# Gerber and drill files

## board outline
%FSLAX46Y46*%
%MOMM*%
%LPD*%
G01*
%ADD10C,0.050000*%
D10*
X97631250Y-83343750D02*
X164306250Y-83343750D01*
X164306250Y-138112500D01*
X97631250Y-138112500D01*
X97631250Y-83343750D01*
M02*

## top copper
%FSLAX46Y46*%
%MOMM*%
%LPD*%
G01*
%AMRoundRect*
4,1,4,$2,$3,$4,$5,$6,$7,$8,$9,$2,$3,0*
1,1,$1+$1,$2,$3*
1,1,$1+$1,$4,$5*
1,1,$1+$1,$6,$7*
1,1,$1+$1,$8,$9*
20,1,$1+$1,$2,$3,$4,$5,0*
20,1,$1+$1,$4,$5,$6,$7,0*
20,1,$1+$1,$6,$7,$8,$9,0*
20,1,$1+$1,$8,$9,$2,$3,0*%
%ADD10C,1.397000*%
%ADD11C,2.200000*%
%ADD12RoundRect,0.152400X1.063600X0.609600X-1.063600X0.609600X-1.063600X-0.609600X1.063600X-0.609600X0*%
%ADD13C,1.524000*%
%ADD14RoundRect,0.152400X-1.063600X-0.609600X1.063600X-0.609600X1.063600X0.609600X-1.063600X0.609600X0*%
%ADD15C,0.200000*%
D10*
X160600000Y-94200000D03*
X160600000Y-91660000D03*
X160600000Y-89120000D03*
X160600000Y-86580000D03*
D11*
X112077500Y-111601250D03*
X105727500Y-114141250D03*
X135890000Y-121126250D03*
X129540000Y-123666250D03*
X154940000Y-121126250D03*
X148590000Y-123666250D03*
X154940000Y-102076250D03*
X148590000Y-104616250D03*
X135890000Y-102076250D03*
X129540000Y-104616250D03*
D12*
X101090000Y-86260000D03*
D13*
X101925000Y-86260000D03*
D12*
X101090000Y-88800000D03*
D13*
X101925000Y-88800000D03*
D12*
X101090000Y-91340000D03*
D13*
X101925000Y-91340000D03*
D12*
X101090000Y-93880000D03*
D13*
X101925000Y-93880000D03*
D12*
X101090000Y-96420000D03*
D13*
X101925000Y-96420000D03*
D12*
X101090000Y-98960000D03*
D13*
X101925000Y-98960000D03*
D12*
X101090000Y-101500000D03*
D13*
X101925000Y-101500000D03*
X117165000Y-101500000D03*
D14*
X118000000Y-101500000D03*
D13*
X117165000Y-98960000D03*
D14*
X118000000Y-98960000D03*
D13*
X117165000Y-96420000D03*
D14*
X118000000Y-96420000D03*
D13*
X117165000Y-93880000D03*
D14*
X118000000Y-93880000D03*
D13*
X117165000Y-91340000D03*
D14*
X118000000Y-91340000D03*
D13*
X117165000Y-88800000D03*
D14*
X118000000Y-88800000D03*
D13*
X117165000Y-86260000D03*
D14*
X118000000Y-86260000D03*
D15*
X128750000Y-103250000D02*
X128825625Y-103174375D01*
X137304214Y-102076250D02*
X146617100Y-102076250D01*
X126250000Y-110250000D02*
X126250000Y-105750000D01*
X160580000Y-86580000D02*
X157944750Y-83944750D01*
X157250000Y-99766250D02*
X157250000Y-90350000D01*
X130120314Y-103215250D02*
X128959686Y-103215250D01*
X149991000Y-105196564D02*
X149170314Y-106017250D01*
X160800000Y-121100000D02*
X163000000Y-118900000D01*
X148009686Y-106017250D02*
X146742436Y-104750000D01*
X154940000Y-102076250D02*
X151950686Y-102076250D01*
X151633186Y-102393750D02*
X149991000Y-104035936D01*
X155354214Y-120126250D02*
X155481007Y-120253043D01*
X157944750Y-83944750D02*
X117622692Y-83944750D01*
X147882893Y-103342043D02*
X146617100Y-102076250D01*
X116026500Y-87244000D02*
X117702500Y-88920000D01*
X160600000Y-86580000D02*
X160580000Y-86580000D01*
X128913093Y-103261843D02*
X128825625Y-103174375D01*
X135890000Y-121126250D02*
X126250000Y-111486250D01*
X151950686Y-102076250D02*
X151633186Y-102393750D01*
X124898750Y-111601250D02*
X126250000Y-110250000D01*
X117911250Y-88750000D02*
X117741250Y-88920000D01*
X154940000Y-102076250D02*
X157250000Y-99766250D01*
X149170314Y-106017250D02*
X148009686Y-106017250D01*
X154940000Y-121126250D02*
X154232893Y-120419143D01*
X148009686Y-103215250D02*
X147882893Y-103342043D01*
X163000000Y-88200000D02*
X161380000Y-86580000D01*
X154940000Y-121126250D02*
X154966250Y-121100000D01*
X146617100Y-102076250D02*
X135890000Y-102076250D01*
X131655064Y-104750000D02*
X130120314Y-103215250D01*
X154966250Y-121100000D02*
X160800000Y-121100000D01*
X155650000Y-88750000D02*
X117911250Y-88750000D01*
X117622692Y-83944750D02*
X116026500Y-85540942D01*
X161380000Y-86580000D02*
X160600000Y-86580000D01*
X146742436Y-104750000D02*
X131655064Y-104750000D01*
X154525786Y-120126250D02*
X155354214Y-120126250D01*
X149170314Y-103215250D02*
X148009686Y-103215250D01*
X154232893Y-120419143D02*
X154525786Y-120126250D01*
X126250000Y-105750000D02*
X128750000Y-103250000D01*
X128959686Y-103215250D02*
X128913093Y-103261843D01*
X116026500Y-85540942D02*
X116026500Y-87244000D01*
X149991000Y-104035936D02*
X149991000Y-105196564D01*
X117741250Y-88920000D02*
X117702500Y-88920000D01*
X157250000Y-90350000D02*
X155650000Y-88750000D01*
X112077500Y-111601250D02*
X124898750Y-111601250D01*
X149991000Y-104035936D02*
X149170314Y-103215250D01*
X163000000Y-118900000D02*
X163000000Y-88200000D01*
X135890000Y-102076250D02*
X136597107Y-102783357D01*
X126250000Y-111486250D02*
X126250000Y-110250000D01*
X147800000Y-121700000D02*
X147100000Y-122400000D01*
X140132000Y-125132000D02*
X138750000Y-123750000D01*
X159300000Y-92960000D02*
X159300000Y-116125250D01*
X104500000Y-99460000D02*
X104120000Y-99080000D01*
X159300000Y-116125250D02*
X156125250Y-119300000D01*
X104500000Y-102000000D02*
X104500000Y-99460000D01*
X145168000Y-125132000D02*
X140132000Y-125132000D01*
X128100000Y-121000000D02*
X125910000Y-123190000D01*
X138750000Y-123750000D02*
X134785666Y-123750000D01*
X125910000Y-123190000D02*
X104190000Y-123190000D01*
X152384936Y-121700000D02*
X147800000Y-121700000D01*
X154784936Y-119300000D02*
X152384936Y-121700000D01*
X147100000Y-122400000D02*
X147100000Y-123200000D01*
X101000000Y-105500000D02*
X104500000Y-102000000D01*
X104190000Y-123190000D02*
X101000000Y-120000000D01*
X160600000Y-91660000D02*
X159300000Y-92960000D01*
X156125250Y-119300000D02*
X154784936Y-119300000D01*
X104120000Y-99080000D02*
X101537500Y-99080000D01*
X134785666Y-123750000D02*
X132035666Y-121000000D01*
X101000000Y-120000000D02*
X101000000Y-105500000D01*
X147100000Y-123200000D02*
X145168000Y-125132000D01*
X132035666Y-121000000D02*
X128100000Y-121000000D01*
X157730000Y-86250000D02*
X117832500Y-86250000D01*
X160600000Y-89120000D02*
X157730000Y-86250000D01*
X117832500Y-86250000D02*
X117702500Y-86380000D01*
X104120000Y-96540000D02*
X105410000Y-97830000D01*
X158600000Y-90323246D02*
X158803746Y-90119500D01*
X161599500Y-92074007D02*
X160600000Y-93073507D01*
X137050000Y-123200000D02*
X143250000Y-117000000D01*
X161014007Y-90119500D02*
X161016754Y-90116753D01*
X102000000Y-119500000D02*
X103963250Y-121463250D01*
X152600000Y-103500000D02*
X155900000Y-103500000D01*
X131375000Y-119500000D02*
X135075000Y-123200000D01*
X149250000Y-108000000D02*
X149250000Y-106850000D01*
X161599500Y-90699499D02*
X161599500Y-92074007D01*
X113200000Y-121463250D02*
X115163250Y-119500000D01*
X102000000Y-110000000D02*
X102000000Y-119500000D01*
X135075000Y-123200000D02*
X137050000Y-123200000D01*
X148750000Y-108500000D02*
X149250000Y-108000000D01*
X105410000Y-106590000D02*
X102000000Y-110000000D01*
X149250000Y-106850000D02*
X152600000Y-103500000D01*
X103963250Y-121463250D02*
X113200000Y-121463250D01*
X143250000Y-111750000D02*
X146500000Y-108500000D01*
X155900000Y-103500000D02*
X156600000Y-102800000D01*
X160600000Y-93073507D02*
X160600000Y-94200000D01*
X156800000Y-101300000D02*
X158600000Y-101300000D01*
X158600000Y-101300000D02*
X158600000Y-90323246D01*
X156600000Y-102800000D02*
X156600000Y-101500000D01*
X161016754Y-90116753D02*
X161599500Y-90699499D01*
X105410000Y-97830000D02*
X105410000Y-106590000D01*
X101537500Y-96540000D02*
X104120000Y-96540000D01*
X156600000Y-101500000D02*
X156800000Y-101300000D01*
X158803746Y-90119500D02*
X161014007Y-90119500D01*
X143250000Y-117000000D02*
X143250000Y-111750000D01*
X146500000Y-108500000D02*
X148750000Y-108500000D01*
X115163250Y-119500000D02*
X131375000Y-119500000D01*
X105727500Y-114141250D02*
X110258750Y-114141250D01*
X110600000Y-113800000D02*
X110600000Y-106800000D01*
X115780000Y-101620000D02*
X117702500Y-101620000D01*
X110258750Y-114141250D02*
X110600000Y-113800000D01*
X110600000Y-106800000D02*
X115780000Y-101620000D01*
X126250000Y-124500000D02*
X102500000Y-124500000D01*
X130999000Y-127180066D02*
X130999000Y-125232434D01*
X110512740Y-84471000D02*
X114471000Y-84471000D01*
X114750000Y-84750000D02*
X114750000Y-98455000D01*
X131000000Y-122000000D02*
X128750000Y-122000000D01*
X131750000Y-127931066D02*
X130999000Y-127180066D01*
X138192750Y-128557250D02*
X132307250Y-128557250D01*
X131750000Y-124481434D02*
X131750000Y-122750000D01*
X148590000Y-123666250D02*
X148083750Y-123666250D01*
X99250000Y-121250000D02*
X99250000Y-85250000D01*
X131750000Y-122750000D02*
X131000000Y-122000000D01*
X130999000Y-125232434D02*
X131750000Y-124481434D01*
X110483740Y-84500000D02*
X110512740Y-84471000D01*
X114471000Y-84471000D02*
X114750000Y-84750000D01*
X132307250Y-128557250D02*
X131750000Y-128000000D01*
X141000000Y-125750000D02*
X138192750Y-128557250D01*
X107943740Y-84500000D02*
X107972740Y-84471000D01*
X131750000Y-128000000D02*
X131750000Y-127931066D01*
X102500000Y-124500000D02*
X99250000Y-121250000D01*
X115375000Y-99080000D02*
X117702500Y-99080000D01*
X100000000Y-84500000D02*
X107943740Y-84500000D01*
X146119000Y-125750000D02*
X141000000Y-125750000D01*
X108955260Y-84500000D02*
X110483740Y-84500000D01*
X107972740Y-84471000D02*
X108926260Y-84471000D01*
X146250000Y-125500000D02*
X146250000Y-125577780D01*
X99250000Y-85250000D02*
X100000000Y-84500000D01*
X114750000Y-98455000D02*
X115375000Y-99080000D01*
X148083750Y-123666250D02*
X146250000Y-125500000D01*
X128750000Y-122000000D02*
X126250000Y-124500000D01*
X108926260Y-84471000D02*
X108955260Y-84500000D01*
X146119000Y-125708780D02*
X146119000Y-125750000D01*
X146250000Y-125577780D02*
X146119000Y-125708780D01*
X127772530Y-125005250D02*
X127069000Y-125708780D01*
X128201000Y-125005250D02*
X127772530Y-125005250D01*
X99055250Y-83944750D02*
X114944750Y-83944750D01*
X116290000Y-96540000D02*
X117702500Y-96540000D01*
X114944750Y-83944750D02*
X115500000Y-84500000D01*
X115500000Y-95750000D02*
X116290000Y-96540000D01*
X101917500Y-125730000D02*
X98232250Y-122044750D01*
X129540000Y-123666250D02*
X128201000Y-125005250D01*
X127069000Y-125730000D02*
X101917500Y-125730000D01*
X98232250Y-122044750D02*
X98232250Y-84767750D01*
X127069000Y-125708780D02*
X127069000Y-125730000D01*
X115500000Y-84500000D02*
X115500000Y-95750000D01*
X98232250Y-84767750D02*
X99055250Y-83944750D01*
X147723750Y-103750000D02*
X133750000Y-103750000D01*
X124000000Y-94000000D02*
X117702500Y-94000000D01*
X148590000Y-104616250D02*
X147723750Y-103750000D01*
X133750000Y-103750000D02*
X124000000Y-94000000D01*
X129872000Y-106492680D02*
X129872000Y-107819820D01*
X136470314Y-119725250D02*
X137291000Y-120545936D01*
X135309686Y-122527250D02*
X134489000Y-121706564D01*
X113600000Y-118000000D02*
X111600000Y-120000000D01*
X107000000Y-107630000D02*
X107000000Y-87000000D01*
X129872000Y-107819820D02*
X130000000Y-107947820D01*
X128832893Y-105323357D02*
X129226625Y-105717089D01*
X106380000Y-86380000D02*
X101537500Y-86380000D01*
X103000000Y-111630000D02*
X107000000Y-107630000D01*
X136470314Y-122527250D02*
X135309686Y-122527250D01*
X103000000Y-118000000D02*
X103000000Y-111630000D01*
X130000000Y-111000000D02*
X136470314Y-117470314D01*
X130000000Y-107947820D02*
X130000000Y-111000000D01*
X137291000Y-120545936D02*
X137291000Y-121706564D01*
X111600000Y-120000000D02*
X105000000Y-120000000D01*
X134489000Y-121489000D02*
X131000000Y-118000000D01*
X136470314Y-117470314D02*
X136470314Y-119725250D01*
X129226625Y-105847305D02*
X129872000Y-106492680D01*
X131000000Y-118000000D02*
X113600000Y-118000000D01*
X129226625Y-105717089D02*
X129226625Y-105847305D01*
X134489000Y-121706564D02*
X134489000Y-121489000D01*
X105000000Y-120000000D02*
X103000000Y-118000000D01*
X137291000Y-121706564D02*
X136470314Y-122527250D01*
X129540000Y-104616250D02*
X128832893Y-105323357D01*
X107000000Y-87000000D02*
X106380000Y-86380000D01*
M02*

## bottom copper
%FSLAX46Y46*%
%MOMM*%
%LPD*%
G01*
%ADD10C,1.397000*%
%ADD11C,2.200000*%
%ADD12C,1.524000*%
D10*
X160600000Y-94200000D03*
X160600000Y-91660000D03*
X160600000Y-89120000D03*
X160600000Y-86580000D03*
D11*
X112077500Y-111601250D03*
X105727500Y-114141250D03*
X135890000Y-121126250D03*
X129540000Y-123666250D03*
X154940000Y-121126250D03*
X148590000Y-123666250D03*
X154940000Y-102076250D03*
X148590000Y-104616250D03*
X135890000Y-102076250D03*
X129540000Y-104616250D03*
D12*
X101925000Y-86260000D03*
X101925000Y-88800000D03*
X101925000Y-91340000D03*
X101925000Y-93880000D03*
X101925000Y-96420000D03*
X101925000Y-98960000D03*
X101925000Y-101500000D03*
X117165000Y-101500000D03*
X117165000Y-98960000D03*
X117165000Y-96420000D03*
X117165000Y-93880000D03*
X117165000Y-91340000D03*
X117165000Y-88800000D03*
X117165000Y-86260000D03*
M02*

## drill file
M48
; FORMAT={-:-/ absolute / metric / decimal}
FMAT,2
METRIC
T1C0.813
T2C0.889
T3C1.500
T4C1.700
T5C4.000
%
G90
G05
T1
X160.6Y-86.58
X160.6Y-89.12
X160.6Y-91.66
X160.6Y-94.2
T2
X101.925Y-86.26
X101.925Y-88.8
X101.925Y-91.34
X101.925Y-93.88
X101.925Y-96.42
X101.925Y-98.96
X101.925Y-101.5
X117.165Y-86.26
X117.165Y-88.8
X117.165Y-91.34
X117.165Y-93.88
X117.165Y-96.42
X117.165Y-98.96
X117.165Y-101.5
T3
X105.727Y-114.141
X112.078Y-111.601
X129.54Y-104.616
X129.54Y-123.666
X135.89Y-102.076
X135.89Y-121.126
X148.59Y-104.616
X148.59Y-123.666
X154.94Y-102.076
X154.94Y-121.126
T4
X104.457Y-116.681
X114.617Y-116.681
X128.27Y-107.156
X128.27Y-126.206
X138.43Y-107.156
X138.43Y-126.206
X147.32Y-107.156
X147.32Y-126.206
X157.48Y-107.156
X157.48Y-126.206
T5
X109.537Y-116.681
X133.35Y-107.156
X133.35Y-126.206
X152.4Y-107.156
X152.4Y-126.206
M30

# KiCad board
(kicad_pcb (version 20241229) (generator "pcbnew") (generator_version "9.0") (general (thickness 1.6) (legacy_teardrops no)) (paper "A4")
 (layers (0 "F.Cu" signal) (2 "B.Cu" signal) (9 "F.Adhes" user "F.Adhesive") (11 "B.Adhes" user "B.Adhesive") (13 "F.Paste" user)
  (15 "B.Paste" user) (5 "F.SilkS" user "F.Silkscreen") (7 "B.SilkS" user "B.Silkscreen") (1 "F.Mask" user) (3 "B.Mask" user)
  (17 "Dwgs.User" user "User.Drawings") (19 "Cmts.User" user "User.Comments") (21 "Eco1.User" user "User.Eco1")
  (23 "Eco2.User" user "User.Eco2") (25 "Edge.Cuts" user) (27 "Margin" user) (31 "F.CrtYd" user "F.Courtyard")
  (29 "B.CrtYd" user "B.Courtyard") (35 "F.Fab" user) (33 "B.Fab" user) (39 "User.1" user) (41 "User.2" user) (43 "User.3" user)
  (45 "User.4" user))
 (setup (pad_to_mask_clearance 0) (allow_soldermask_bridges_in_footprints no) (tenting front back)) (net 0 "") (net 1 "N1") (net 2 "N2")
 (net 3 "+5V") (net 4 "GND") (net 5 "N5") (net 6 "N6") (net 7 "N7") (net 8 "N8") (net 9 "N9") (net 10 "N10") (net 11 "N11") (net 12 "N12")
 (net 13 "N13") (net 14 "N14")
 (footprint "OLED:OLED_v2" (layer "F.Cu") (at 160.6 90.39 90)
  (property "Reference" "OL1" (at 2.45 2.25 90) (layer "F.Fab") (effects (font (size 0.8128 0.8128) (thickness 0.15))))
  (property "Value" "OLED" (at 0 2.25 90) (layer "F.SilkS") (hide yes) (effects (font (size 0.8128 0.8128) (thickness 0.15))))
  (pad "1" thru_hole circle (at -3.81 0 90) (size 1.397 1.397) (drill 0.8128) (layers "*.Cu" "B.Mask" "F.SilkS") (remove_unused_layers no)
   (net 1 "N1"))
  (pad "2" thru_hole circle (at -1.27 0 90) (size 1.397 1.397) (drill 0.8128) (layers "*.Cu" "B.Mask" "F.SilkS") (remove_unused_layers no)
   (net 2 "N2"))
  (pad "3" thru_hole circle (at 1.27 0 90) (size 1.397 1.397) (drill 0.8128) (layers "*.Cu" "B.Mask" "F.SilkS") (remove_unused_layers no)
   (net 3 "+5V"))
  (pad "4" thru_hole circle (at 3.81 0 90) (size 1.397 1.397) (drill 0.8128) (layers "*.Cu" "B.Mask" "F.SilkS") (remove_unused_layers no)
   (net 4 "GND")))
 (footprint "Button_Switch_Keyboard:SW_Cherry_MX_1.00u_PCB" (layer "F.Cu") (at 112.0775 111.60125)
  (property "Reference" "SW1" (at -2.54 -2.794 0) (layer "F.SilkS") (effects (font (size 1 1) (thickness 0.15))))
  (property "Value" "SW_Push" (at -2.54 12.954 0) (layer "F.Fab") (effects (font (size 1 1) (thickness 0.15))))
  (pad "" np_thru_hole circle (at -7.62 5.08) (size 1.7 1.7) (drill 1.7) (layers "*.Cu" "*.Mask"))
  (pad "" np_thru_hole circle (at -2.54 5.08) (size 4 4) (drill 4) (layers "*.Cu" "*.Mask"))
  (pad "" np_thru_hole circle (at 2.54 5.08) (size 1.7 1.7) (drill 1.7) (layers "*.Cu" "*.Mask"))
  (pad "1" thru_hole circle (at 0 0) (size 2.2 2.2) (drill 1.5) (layers "*.Cu" "*.Mask") (remove_unused_layers no) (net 4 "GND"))
  (pad "2" thru_hole circle (at -6.35 2.54) (size 2.2 2.2) (drill 1.5) (layers "*.Cu" "*.Mask") (remove_unused_layers no) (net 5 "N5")))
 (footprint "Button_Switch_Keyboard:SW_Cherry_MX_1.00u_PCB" (layer "F.Cu") (at 135.89 121.12625)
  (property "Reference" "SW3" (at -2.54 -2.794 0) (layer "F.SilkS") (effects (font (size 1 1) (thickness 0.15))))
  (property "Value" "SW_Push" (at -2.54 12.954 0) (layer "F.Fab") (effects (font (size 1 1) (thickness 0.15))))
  (pad "" np_thru_hole circle (at -7.62 5.08) (size 1.7 1.7) (drill 1.7) (layers "*.Cu" "*.Mask"))
  (pad "" np_thru_hole circle (at -2.54 5.08) (size 4 4) (drill 4) (layers "*.Cu" "*.Mask"))
  (pad "" np_thru_hole circle (at 2.54 5.08) (size 1.7 1.7) (drill 1.7) (layers "*.Cu" "*.Mask"))
  (pad "1" thru_hole circle (at 0 0) (size 2.2 2.2) (drill 1.5) (layers "*.Cu" "*.Mask") (remove_unused_layers no) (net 4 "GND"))
  (pad "2" thru_hole circle (at -6.35 2.54) (size 2.2 2.2) (drill 1.5) (layers "*.Cu" "*.Mask") (remove_unused_layers no) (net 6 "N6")))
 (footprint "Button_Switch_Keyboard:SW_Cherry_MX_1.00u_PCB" (layer "F.Cu") (at 154.94 121.12625)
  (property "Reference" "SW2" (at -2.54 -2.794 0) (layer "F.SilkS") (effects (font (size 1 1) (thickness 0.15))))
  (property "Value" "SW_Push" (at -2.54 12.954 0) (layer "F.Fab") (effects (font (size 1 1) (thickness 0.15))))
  (pad "" np_thru_hole circle (at -7.62 5.08) (size 1.7 1.7) (drill 1.7) (layers "*.Cu" "*.Mask"))
  (pad "" np_thru_hole circle (at -2.54 5.08) (size 4 4) (drill 4) (layers "*.Cu" "*.Mask"))
  (pad "" np_thru_hole circle (at 2.54 5.08) (size 1.7 1.7) (drill 1.7) (layers "*.Cu" "*.Mask"))
  (pad "1" thru_hole circle (at 0 0) (size 2.2 2.2) (drill 1.5) (layers "*.Cu" "*.Mask") (remove_unused_layers no) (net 4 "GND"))
  (pad "2" thru_hole circle (at -6.35 2.54) (size 2.2 2.2) (drill 1.5) (layers "*.Cu" "*.Mask") (remove_unused_layers no) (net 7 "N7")))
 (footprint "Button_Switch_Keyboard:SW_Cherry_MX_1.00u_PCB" (layer "F.Cu") (at 154.94 102.07625)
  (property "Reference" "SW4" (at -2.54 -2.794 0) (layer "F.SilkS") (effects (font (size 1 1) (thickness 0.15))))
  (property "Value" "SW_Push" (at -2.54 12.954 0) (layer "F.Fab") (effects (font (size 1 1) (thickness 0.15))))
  (pad "" np_thru_hole circle (at -7.62 5.08) (size 1.7 1.7) (drill 1.7) (layers "*.Cu" "*.Mask"))
  (pad "" np_thru_hole circle (at -2.54 5.08) (size 4 4) (drill 4) (layers "*.Cu" "*.Mask"))
  (pad "" np_thru_hole circle (at 2.54 5.08) (size 1.7 1.7) (drill 1.7) (layers "*.Cu" "*.Mask"))
  (pad "1" thru_hole circle (at 0 0) (size 2.2 2.2) (drill 1.5) (layers "*.Cu" "*.Mask") (remove_unused_layers no) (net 4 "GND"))
  (pad "2" thru_hole circle (at -6.35 2.54) (size 2.2 2.2) (drill 1.5) (layers "*.Cu" "*.Mask") (remove_unused_layers no) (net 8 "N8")))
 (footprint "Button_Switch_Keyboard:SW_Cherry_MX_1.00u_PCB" (layer "F.Cu") (at 135.89 102.07625)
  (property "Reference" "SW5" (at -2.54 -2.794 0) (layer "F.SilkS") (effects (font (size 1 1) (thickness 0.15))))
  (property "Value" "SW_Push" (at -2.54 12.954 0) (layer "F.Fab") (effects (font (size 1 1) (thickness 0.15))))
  (pad "" np_thru_hole circle (at -7.62 5.08) (size 1.7 1.7) (drill 1.7) (layers "*.Cu" "*.Mask"))
  (pad "" np_thru_hole circle (at -2.54 5.08) (size 4 4) (drill 4) (layers "*.Cu" "*.Mask"))
  (pad "" np_thru_hole circle (at 2.54 5.08) (size 1.7 1.7) (drill 1.7) (layers "*.Cu" "*.Mask"))
  (pad "1" thru_hole circle (at 0 0) (size 2.2 2.2) (drill 1.5) (layers "*.Cu" "*.Mask") (remove_unused_layers no) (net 4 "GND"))
  (pad "2" thru_hole circle (at -6.35 2.54) (size 2.2 2.2) (drill 1.5) (layers "*.Cu" "*.Mask") (remove_unused_layers no) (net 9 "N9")))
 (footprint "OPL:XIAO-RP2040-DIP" (layer "F.Cu") (at 109.545 93.88)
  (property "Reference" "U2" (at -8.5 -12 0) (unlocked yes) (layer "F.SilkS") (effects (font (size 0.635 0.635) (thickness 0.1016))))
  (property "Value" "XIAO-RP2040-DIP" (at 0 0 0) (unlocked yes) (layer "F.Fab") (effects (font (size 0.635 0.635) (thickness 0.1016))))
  (pad "1" smd roundrect (at -8.455 -7.62 180) (size 2.432 1.524) (layers "F.Cu" "F.Mask") (roundrect_rratio 0.1) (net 9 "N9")
   (thermal_bridge_angle 45))
  (pad "1" thru_hole circle (at -7.62 -7.62 180) (size 1.524 1.524) (drill 0.889) (layers "*.Cu" "*.Mask") (remove_unused_layers no)
   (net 9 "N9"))
  (pad "2" smd roundrect (at -8.455 -5.08 180) (size 2.432 1.524) (layers "F.Cu" "F.Mask") (roundrect_rratio 0.1) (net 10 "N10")
   (thermal_bridge_angle 45))
  (pad "2" thru_hole circle (at -7.62 -5.08 180) (size 1.524 1.524) (drill 0.889) (layers "*.Cu" "*.Mask") (remove_unused_layers no)
   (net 10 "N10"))
  (pad "3" smd roundrect (at -8.455 -2.54 180) (size 2.432 1.524) (layers "F.Cu" "F.Mask") (roundrect_rratio 0.1) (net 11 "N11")
   (thermal_bridge_angle 45))
  (pad "3" thru_hole circle (at -7.62 -2.54 180) (size 1.524 1.524) (drill 0.889) (layers "*.Cu" "*.Mask") (remove_unused_layers no)
   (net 11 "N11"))
  (pad "4" smd roundrect (at -8.455 0 180) (size 2.432 1.524) (layers "F.Cu" "F.Mask") (roundrect_rratio 0.1) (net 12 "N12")
   (thermal_bridge_angle 45))
  (pad "4" thru_hole circle (at -7.62 0 180) (size 1.524 1.524) (drill 0.889) (layers "*.Cu" "*.Mask") (remove_unused_layers no)
   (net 12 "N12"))
  (pad "5" smd roundrect (at -8.455 2.54 180) (size 2.432 1.524) (layers "F.Cu" "F.Mask") (roundrect_rratio 0.1) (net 1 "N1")
   (thermal_bridge_angle 45))
  (pad "5" thru_hole circle (at -7.62 2.54 180) (size 1.524 1.524) (drill 0.889) (layers "*.Cu" "*.Mask") (remove_unused_layers no)
   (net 1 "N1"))
  (pad "6" smd roundrect (at -8.455 5.08 180) (size 2.432 1.524) (layers "F.Cu" "F.Mask") (roundrect_rratio 0.1) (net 2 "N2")
   (thermal_bridge_angle 45))
  (pad "6" thru_hole circle (at -7.62 5.08 180) (size 1.524 1.524) (drill 0.889) (layers "*.Cu" "*.Mask") (remove_unused_layers no)
   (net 2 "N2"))
  (pad "7" smd roundrect (at -8.455 7.62 180) (size 2.432 1.524) (layers "F.Cu" "F.Mask") (roundrect_rratio 0.1) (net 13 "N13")
   (thermal_bridge_angle 45))
  (pad "7" thru_hole circle (at -7.62 7.62 180) (size 1.524 1.524) (drill 0.889) (layers "*.Cu" "*.Mask") (remove_unused_layers no)
   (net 13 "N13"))
  (pad "8" thru_hole circle (at 7.62 7.62) (size 1.524 1.524) (drill 0.889) (layers "*.Cu" "*.Mask") (remove_unused_layers no) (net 5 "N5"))
  (pad "8" smd roundrect (at 8.455 7.62) (size 2.432 1.524) (layers "F.Cu" "F.Mask") (roundrect_rratio 0.1) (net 5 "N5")
   (thermal_bridge_angle 45))
  (pad "9" thru_hole circle (at 7.62 5.08) (size 1.524 1.524) (drill 0.889) (layers "*.Cu" "*.Mask") (remove_unused_layers no) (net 7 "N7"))
  (pad "9" smd roundrect (at 8.455 5.08) (size 2.432 1.524) (layers "F.Cu" "F.Mask") (roundrect_rratio 0.1) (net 7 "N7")
   (thermal_bridge_angle 45))
  (pad "10" thru_hole circle (at 7.62 2.54) (size 1.524 1.524) (drill 0.889) (layers "*.Cu" "*.Mask") (remove_unused_layers no) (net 6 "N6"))
  (pad "10" smd roundrect (at 8.455 2.54) (size 2.432 1.524) (layers "F.Cu" "F.Mask") (roundrect_rratio 0.1) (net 6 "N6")
   (thermal_bridge_angle 45))
  (pad "11" thru_hole circle (at 7.62 0) (size 1.524 1.524) (drill 0.889) (layers "*.Cu" "*.Mask") (remove_unused_layers no) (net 8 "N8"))
  (pad "11" smd roundrect (at 8.455 0) (size 2.432 1.524) (layers "F.Cu" "F.Mask") (roundrect_rratio 0.1) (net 8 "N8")
   (thermal_bridge_angle 45))
  (pad "12" thru_hole circle (at 7.62 -2.54) (size 1.524 1.524) (drill 0.889) (layers "*.Cu" "*.Mask") (remove_unused_layers no)
   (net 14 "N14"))
  (pad "12" smd roundrect (at 8.455 -2.54) (size 2.432 1.524) (layers "F.Cu" "F.Mask") (roundrect_rratio 0.1) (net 14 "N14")
   (thermal_bridge_angle 45))
  (pad "13" thru_hole circle (at 7.62 -5.08) (size 1.524 1.524) (drill 0.889) (layers "*.Cu" "*.Mask") (remove_unused_layers no)
   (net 4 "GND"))
  (pad "13" smd roundrect (at 8.455 -5.08) (size 2.432 1.524) (layers "F.Cu" "F.Mask") (roundrect_rratio 0.1) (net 4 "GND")
   (thermal_bridge_angle 45))
  (pad "14" thru_hole circle (at 7.62 -7.62) (size 1.524 1.524) (drill 0.889) (layers "*.Cu" "*.Mask") (remove_unused_layers no)
   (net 3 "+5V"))
  (pad "14" smd roundrect (at 8.455 -7.62) (size 2.432 1.524) (layers "F.Cu" "F.Mask") (roundrect_rratio 0.1) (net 3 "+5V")
   (thermal_bridge_angle 45)))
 (gr_rect (start 97.63125 83.34375) (end 164.30625 138.1125) (stroke (width 0.05) (type default)) (fill no) (layer "Edge.Cuts"))
 (segment (start 128.75 103.25) (end 128.825625 103.174375) (width 0.2) (layer "F.Cu") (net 4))
 (segment (start 137.304214 102.07625) (end 146.6171 102.07625) (width 0.2) (layer "F.Cu") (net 4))
 (segment (start 126.25 110.25) (end 126.25 105.75) (width 0.2) (layer "F.Cu") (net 4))
 (segment (start 160.58 86.58) (end 157.94475 83.94475) (width 0.2) (layer "F.Cu") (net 4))
 (segment (start 157.25 99.76625) (end 157.25 90.35) (width 0.2) (layer "F.Cu") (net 4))
 (segment (start 130.120314 103.21525) (end 128.959686 103.21525) (width 0.2) (layer "F.Cu") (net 4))
 (segment (start 149.991 105.196564) (end 149.170314 106.01725) (width 0.2) (layer "F.Cu") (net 4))
 (segment (start 160.8 121.1) (end 163 118.9) (width 0.2) (layer "F.Cu") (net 4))
 (segment (start 148.009686 106.01725) (end 146.742436 104.75) (width 0.2) (layer "F.Cu") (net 4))
 (segment (start 154.94 102.07625) (end 151.950686 102.07625) (width 0.2) (layer "F.Cu") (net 4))
 (segment (start 151.633186 102.39375) (end 149.991 104.035936) (width 0.2) (layer "F.Cu") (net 4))
 (segment (start 155.354214 120.12625) (end 155.481007 120.253043) (width 0.2) (layer "F.Cu") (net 4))
 (segment (start 157.94475 83.94475) (end 117.622692 83.94475) (width 0.2) (layer "F.Cu") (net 4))
 (segment (start 147.882893 103.342043) (end 146.6171 102.07625) (width 0.2) (layer "F.Cu") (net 4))
 (segment (start 116.0265 87.244) (end 117.7025 88.92) (width 0.2) (layer "F.Cu") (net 4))
 (segment (start 160.6 86.58) (end 160.58 86.58) (width 0.2) (layer "F.Cu") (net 4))
 (segment (start 128.913093 103.261843) (end 128.825625 103.174375) (width 0.2) (layer "F.Cu") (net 4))
 (segment (start 135.89 121.12625) (end 126.25 111.48625) (width 0.2) (layer "F.Cu") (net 4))
 (segment (start 151.950686 102.07625) (end 151.633186 102.39375) (width 0.2) (layer "F.Cu") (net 4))
 (segment (start 124.89875 111.60125) (end 126.25 110.25) (width 0.2) (layer "F.Cu") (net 4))
 (segment (start 117.91125 88.75) (end 117.74125 88.92) (width 0.2) (layer "F.Cu") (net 4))
 (segment (start 154.94 102.07625) (end 157.25 99.76625) (width 0.2) (layer "F.Cu") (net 4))
 (segment (start 149.170314 106.01725) (end 148.009686 106.01725) (width 0.2) (layer "F.Cu") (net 4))
 (segment (start 154.94 121.12625) (end 154.232893 120.419143) (width 0.2) (layer "F.Cu") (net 4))
 (segment (start 148.009686 103.21525) (end 147.882893 103.342043) (width 0.2) (layer "F.Cu") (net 4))
 (segment (start 163 88.2) (end 161.38 86.58) (width 0.2) (layer "F.Cu") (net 4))
 (segment (start 154.94 121.12625) (end 154.96625 121.1) (width 0.2) (layer "F.Cu") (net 4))
 (segment (start 146.6171 102.07625) (end 135.89 102.07625) (width 0.2) (layer "F.Cu") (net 4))
 (segment (start 131.655064 104.75) (end 130.120314 103.21525) (width 0.2) (layer "F.Cu") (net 4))
 (segment (start 154.96625 121.1) (end 160.8 121.1) (width 0.2) (layer "F.Cu") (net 4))
 (segment (start 155.65 88.75) (end 117.91125 88.75) (width 0.2) (layer "F.Cu") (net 4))
 (segment (start 117.622692 83.94475) (end 116.0265 85.540942) (width 0.2) (layer "F.Cu") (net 4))
 (segment (start 161.38 86.58) (end 160.6 86.58) (width 0.2) (layer "F.Cu") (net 4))
 (segment (start 146.742436 104.75) (end 131.655064 104.75) (width 0.2) (layer "F.Cu") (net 4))
 (segment (start 154.525786 120.12625) (end 155.354214 120.12625) (width 0.2) (layer "F.Cu") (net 4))
 (segment (start 149.170314 103.21525) (end 148.009686 103.21525) (width 0.2) (layer "F.Cu") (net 4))
 (segment (start 154.232893 120.419143) (end 154.525786 120.12625) (width 0.2) (layer "F.Cu") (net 4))
 (segment (start 126.25 105.75) (end 128.75 103.25) (width 0.2) (layer "F.Cu") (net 4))
 (segment (start 128.959686 103.21525) (end 128.913093 103.261843) (width 0.2) (layer "F.Cu") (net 4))
 (segment (start 116.0265 85.540942) (end 116.0265 87.244) (width 0.2) (layer "F.Cu") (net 4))
 (segment (start 149.991 104.035936) (end 149.991 105.196564) (width 0.2) (layer "F.Cu") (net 4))
 (segment (start 117.74125 88.92) (end 117.7025 88.92) (width 0.2) (layer "F.Cu") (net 4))
 (segment (start 157.25 90.35) (end 155.65 88.75) (width 0.2) (layer "F.Cu") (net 4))
 (segment (start 112.0775 111.60125) (end 124.89875 111.60125) (width 0.2) (layer "F.Cu") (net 4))
 (segment (start 149.991 104.035936) (end 149.170314 103.21525) (width 0.2) (layer "F.Cu") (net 4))
 (segment (start 163 118.9) (end 163 88.2) (width 0.2) (layer "F.Cu") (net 4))
 (segment (start 135.89 102.07625) (end 136.597107 102.783357) (width 0.2) (layer "F.Cu") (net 4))
 (segment (start 126.25 111.48625) (end 126.25 110.25) (width 0.2) (layer "F.Cu") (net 4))
 (segment (start 147.8 121.7) (end 147.1 122.4) (width 0.2) (layer "F.Cu") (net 2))
 (segment (start 140.132 125.132) (end 138.75 123.75) (width 0.2) (layer "F.Cu") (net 2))
 (segment (start 159.3 92.96) (end 159.3 116.12525) (width 0.2) (layer "F.Cu") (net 2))
 (segment (start 104.5 99.46) (end 104.12 99.08) (width 0.2) (layer "F.Cu") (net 2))
 (segment (start 159.3 116.12525) (end 156.12525 119.3) (width 0.2) (layer "F.Cu") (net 2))
 (segment (start 104.5 102) (end 104.5 99.46) (width 0.2) (layer "F.Cu") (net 2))
 (segment (start 145.168 125.132) (end 140.132 125.132) (width 0.2) (layer "F.Cu") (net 2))
 (segment (start 128.1 121) (end 125.91 123.19) (width 0.2) (layer "F.Cu") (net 2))
 (segment (start 138.75 123.75) (end 134.785666 123.75) (width 0.2) (layer "F.Cu") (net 2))
 (segment (start 125.91 123.19) (end 104.19 123.19) (width 0.2) (layer "F.Cu") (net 2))
 (segment (start 152.384936 121.7) (end 147.8 121.7) (width 0.2) (layer "F.Cu") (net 2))
 (segment (start 154.784936 119.3) (end 152.384936 121.7) (width 0.2) (layer "F.Cu") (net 2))
 (segment (start 147.1 122.4) (end 147.1 123.2) (width 0.2) (layer "F.Cu") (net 2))
 (segment (start 101 105.5) (end 104.5 102) (width 0.2) (layer "F.Cu") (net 2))
 (segment (start 104.19 123.19) (end 101 120) (width 0.2) (layer "F.Cu") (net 2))
 (segment (start 160.6 91.66) (end 159.3 92.96) (width 0.2) (layer "F.Cu") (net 2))
 (segment (start 156.12525 119.3) (end 154.784936 119.3) (width 0.2) (layer "F.Cu") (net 2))
 (segment (start 104.12 99.08) (end 101.5375 99.08) (width 0.2) (layer "F.Cu") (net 2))
 (segment (start 134.785666 123.75) (end 132.035666 121) (width 0.2) (layer "F.Cu") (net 2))
 (segment (start 101 120) (end 101 105.5) (width 0.2) (layer "F.Cu") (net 2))
 (segment (start 147.1 123.2) (end 145.168 125.132) (width 0.2) (layer "F.Cu") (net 2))
 (segment (start 132.035666 121) (end 128.1 121) (width 0.2) (layer "F.Cu") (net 2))
 (segment (start 157.73 86.25) (end 117.8325 86.25) (width 0.2) (layer "F.Cu") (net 3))
 (segment (start 160.6 89.12) (end 157.73 86.25) (width 0.2) (layer "F.Cu") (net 3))
 (segment (start 117.8325 86.25) (end 117.7025 86.38) (width 0.2) (layer "F.Cu") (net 3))
 (segment (start 104.12 96.54) (end 105.41 97.83) (width 0.2) (layer "F.Cu") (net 1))
 (segment (start 158.6 90.323246) (end 158.803746 90.1195) (width 0.2) (layer "F.Cu") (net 1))
 (segment (start 161.5995 92.074007) (end 160.6 93.073507) (width 0.2) (layer "F.Cu") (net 1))
 (segment (start 137.05 123.2) (end 143.25 117) (width 0.2) (layer "F.Cu") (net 1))
 (segment (start 161.014007 90.1195) (end 161.016754 90.116753) (width 0.2) (layer "F.Cu") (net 1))
 (segment (start 102 119.5) (end 103.96325 121.46325) (width 0.2) (layer "F.Cu") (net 1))
 (segment (start 152.6 103.5) (end 155.9 103.5) (width 0.2) (layer "F.Cu") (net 1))
 (segment (start 131.375 119.5) (end 135.075 123.2) (width 0.2) (layer "F.Cu") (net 1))
 (segment (start 149.25 108) (end 149.25 106.85) (width 0.2) (layer "F.Cu") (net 1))
 (segment (start 161.5995 90.699499) (end 161.5995 92.074007) (width 0.2) (layer "F.Cu") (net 1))
 (segment (start 113.2 121.46325) (end 115.16325 119.5) (width 0.2) (layer "F.Cu") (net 1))
 (segment (start 102 110) (end 102 119.5) (width 0.2) (layer "F.Cu") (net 1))
 (segment (start 135.075 123.2) (end 137.05 123.2) (width 0.2) (layer "F.Cu") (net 1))
 (segment (start 148.75 108.5) (end 149.25 108) (width 0.2) (layer "F.Cu") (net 1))
 (segment (start 105.41 106.59) (end 102 110) (width 0.2) (layer "F.Cu") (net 1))
 (segment (start 149.25 106.85) (end 152.6 103.5) (width 0.2) (layer "F.Cu") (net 1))
 (segment (start 103.96325 121.46325) (end 113.2 121.46325) (width 0.2) (layer "F.Cu") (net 1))
 (segment (start 143.25 111.75) (end 146.5 108.5) (width 0.2) (layer "F.Cu") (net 1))
 (segment (start 155.9 103.5) (end 156.6 102.8) (width 0.2) (layer "F.Cu") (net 1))
 (segment (start 160.6 93.073507) (end 160.6 94.2) (width 0.2) (layer "F.Cu") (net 1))
 (segment (start 156.8 101.3) (end 158.6 101.3) (width 0.2) (layer "F.Cu") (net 1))
 (segment (start 158.6 101.3) (end 158.6 90.323246) (width 0.2) (layer "F.Cu") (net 1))
 (segment (start 156.6 102.8) (end 156.6 101.5) (width 0.2) (layer "F.Cu") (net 1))
 (segment (start 161.016754 90.116753) (end 161.5995 90.699499) (width 0.2) (layer "F.Cu") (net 1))
 (segment (start 105.41 97.83) (end 105.41 106.59) (width 0.2) (layer "F.Cu") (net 1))
 (segment (start 101.5375 96.54) (end 104.12 96.54) (width 0.2) (layer "F.Cu") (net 1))
 (segment (start 156.6 101.5) (end 156.8 101.3) (width 0.2) (layer "F.Cu") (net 1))
 (segment (start 158.803746 90.1195) (end 161.014007 90.1195) (width 0.2) (layer "F.Cu") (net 1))
 (segment (start 143.25 117) (end 143.25 111.75) (width 0.2) (layer "F.Cu") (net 1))
 (segment (start 146.5 108.5) (end 148.75 108.5) (width 0.2) (layer "F.Cu") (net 1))
 (segment (start 115.16325 119.5) (end 131.375 119.5) (width 0.2) (layer "F.Cu") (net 1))
 (segment (start 105.7275 114.14125) (end 110.25875 114.14125) (width 0.2) (layer "F.Cu") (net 5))
 (segment (start 110.6 113.8) (end 110.6 106.8) (width 0.2) (layer "F.Cu") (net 5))
 (segment (start 115.78 101.62) (end 117.7025 101.62) (width 0.2) (layer "F.Cu") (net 5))
 (segment (start 110.25875 114.14125) (end 110.6 113.8) (width 0.2) (layer "F.Cu") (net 5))
 (segment (start 110.6 106.8) (end 115.78 101.62) (width 0.2) (layer "F.Cu") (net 5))
 (segment (start 126.25 124.5) (end 102.5 124.5) (width 0.2) (layer "F.Cu") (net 7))
 (segment (start 130.999 127.180066) (end 130.999 125.232434) (width 0.2) (layer "F.Cu") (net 7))
 (segment (start 110.51274 84.471) (end 114.471 84.471) (width 0.2) (layer "F.Cu") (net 7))
 (segment (start 114.75 84.75) (end 114.75 98.455) (width 0.2) (layer "F.Cu") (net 7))
 (segment (start 131 122) (end 128.75 122) (width 0.2) (layer "F.Cu") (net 7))
 (segment (start 131.75 127.931066) (end 130.999 127.180066) (width 0.2) (layer "F.Cu") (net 7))
 (segment (start 138.19275 128.55725) (end 132.30725 128.55725) (width 0.2) (layer "F.Cu") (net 7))
 (segment (start 131.75 124.481434) (end 131.75 122.75) (width 0.2) (layer "F.Cu") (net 7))
 (segment (start 148.59 123.66625) (end 148.08375 123.66625) (width 0.2) (layer "F.Cu") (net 7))
 (segment (start 99.25 121.25) (end 99.25 85.25) (width 0.2) (layer "F.Cu") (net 7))
 (segment (start 131.75 122.75) (end 131 122) (width 0.2) (layer "F.Cu") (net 7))
 (segment (start 130.999 125.232434) (end 131.75 124.481434) (width 0.2) (layer "F.Cu") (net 7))
 (segment (start 110.48374 84.5) (end 110.51274 84.471) (width 0.2) (layer "F.Cu") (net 7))
 (segment (start 114.471 84.471) (end 114.75 84.75) (width 0.2) (layer "F.Cu") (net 7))
 (segment (start 132.30725 128.55725) (end 131.75 128) (width 0.2) (layer "F.Cu") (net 7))
 (segment (start 141 125.75) (end 138.19275 128.55725) (width 0.2) (layer "F.Cu") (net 7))
 (segment (start 107.94374 84.5) (end 107.97274 84.471) (width 0.2) (layer "F.Cu") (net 7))
 (segment (start 131.75 128) (end 131.75 127.931066) (width 0.2) (layer "F.Cu") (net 7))
 (segment (start 102.5 124.5) (end 99.25 121.25) (width 0.2) (layer "F.Cu") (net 7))
 (segment (start 115.375 99.08) (end 117.7025 99.08) (width 0.2) (layer "F.Cu") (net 7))
 (segment (start 100 84.5) (end 107.94374 84.5) (width 0.2) (layer "F.Cu") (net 7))
 (segment (start 146.119 125.75) (end 141 125.75) (width 0.2) (layer "F.Cu") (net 7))
 (segment (start 108.95526 84.5) (end 110.48374 84.5) (width 0.2) (layer "F.Cu") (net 7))
 (segment (start 107.97274 84.471) (end 108.92626 84.471) (width 0.2) (layer "F.Cu") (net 7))
 (segment (start 146.25 125.5) (end 146.25 125.57778) (width 0.2) (layer "F.Cu") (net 7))
 (segment (start 99.25 85.25) (end 100 84.5) (width 0.2) (layer "F.Cu") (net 7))
 (segment (start 114.75 98.455) (end 115.375 99.08) (width 0.2) (layer "F.Cu") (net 7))
 (segment (start 148.08375 123.66625) (end 146.25 125.5) (width 0.2) (layer "F.Cu") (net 7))
 (segment (start 128.75 122) (end 126.25 124.5) (width 0.2) (layer "F.Cu") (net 7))
 (segment (start 108.92626 84.471) (end 108.95526 84.5) (width 0.2) (layer "F.Cu") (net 7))
 (segment (start 146.119 125.70878) (end 146.119 125.75) (width 0.2) (layer "F.Cu") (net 7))
 (segment (start 146.25 125.57778) (end 146.119 125.70878) (width 0.2) (layer "F.Cu") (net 7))
 (segment (start 127.77253 125.00525) (end 127.069 125.70878) (width 0.2) (layer "F.Cu") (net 6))
 (segment (start 128.201 125.00525) (end 127.77253 125.00525) (width 0.2) (layer "F.Cu") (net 6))
 (segment (start 99.05525 83.94475) (end 114.94475 83.94475) (width 0.2) (layer "F.Cu") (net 6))
 (segment (start 116.29 96.54) (end 117.7025 96.54) (width 0.2) (layer "F.Cu") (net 6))
 (segment (start 114.94475 83.94475) (end 115.5 84.5) (width 0.2) (layer "F.Cu") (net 6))
 (segment (start 115.5 95.75) (end 116.29 96.54) (width 0.2) (layer "F.Cu") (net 6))
 (segment (start 101.9175 125.73) (end 98.23225 122.04475) (width 0.2) (layer "F.Cu") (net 6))
 (segment (start 129.54 123.66625) (end 128.201 125.00525) (width 0.2) (layer "F.Cu") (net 6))
 (segment (start 127.069 125.73) (end 101.9175 125.73) (width 0.2) (layer "F.Cu") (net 6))
 (segment (start 98.23225 122.04475) (end 98.23225 84.76775) (width 0.2) (layer "F.Cu") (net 6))
 (segment (start 127.069 125.70878) (end 127.069 125.73) (width 0.2) (layer "F.Cu") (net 6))
 (segment (start 115.5 84.5) (end 115.5 95.75) (width 0.2) (layer "F.Cu") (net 6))
 (segment (start 98.23225 84.76775) (end 99.05525 83.94475) (width 0.2) (layer "F.Cu") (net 6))
 (segment (start 147.72375 103.75) (end 133.75 103.75) (width 0.2) (layer "F.Cu") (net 8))
 (segment (start 124 94) (end 117.7025 94) (width 0.2) (layer "F.Cu") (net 8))
 (segment (start 148.59 104.61625) (end 147.72375 103.75) (width 0.2) (layer "F.Cu") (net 8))
 (segment (start 133.75 103.75) (end 124 94) (width 0.2) (layer "F.Cu") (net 8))
 (segment (start 129.872 106.49268) (end 129.872 107.81982) (width 0.2) (layer "F.Cu") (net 9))
 (segment (start 136.470314 119.72525) (end 137.291 120.545936) (width 0.2) (layer "F.Cu") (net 9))
 (segment (start 135.309686 122.52725) (end 134.489 121.706564) (width 0.2) (layer "F.Cu") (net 9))
 (segment (start 113.6 118) (end 111.6 120) (width 0.2) (layer "F.Cu") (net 9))
 (segment (start 107 107.63) (end 107 87) (width 0.2) (layer "F.Cu") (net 9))
 (segment (start 129.872 107.81982) (end 130 107.94782) (width 0.2) (layer "F.Cu") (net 9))
 (segment (start 128.832893 105.323357) (end 129.226625 105.717089) (width 0.2) (layer "F.Cu") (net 9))
 (segment (start 106.38 86.38) (end 101.5375 86.38) (width 0.2) (layer "F.Cu") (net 9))
 (segment (start 103 111.63) (end 107 107.63) (width 0.2) (layer "F.Cu") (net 9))
 (segment (start 136.470314 122.52725) (end 135.309686 122.52725) (width 0.2) (layer "F.Cu") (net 9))
 (segment (start 103 118) (end 103 111.63) (width 0.2) (layer "F.Cu") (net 9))
 (segment (start 130 111) (end 136.470314 117.470314) (width 0.2) (layer "F.Cu") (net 9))
 (segment (start 130 107.94782) (end 130 111) (width 0.2) (layer "F.Cu") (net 9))
 (segment (start 137.291 120.545936) (end 137.291 121.706564) (width 0.2) (layer "F.Cu") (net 9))
 (segment (start 111.6 120) (end 105 120) (width 0.2) (layer "F.Cu") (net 9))
 (segment (start 134.489 121.489) (end 131 118) (width 0.2) (layer "F.Cu") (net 9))
 (segment (start 136.470314 117.470314) (end 136.470314 119.72525) (width 0.2) (layer "F.Cu") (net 9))
 (segment (start 129.226625 105.847305) (end 129.872 106.49268) (width 0.2) (layer "F.Cu") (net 9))
 (segment (start 131 118) (end 113.6 118) (width 0.2) (layer "F.Cu") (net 9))
 (segment (start 129.226625 105.717089) (end 129.226625 105.847305) (width 0.2) (layer "F.Cu") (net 9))
 (segment (start 134.489 121.706564) (end 134.489 121.489) (width 0.2) (layer "F.Cu") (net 9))
 (segment (start 105 120) (end 103 118) (width 0.2) (layer "F.Cu") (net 9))
 (segment (start 137.291 121.706564) (end 136.470314 122.52725) (width 0.2) (layer "F.Cu") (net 9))
 (segment (start 129.54 104.61625) (end 128.832893 105.323357) (width 0.2) (layer "F.Cu") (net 9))
 (segment (start 107 87) (end 106.38 86.38) (width 0.2) (layer "F.Cu") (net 9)))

